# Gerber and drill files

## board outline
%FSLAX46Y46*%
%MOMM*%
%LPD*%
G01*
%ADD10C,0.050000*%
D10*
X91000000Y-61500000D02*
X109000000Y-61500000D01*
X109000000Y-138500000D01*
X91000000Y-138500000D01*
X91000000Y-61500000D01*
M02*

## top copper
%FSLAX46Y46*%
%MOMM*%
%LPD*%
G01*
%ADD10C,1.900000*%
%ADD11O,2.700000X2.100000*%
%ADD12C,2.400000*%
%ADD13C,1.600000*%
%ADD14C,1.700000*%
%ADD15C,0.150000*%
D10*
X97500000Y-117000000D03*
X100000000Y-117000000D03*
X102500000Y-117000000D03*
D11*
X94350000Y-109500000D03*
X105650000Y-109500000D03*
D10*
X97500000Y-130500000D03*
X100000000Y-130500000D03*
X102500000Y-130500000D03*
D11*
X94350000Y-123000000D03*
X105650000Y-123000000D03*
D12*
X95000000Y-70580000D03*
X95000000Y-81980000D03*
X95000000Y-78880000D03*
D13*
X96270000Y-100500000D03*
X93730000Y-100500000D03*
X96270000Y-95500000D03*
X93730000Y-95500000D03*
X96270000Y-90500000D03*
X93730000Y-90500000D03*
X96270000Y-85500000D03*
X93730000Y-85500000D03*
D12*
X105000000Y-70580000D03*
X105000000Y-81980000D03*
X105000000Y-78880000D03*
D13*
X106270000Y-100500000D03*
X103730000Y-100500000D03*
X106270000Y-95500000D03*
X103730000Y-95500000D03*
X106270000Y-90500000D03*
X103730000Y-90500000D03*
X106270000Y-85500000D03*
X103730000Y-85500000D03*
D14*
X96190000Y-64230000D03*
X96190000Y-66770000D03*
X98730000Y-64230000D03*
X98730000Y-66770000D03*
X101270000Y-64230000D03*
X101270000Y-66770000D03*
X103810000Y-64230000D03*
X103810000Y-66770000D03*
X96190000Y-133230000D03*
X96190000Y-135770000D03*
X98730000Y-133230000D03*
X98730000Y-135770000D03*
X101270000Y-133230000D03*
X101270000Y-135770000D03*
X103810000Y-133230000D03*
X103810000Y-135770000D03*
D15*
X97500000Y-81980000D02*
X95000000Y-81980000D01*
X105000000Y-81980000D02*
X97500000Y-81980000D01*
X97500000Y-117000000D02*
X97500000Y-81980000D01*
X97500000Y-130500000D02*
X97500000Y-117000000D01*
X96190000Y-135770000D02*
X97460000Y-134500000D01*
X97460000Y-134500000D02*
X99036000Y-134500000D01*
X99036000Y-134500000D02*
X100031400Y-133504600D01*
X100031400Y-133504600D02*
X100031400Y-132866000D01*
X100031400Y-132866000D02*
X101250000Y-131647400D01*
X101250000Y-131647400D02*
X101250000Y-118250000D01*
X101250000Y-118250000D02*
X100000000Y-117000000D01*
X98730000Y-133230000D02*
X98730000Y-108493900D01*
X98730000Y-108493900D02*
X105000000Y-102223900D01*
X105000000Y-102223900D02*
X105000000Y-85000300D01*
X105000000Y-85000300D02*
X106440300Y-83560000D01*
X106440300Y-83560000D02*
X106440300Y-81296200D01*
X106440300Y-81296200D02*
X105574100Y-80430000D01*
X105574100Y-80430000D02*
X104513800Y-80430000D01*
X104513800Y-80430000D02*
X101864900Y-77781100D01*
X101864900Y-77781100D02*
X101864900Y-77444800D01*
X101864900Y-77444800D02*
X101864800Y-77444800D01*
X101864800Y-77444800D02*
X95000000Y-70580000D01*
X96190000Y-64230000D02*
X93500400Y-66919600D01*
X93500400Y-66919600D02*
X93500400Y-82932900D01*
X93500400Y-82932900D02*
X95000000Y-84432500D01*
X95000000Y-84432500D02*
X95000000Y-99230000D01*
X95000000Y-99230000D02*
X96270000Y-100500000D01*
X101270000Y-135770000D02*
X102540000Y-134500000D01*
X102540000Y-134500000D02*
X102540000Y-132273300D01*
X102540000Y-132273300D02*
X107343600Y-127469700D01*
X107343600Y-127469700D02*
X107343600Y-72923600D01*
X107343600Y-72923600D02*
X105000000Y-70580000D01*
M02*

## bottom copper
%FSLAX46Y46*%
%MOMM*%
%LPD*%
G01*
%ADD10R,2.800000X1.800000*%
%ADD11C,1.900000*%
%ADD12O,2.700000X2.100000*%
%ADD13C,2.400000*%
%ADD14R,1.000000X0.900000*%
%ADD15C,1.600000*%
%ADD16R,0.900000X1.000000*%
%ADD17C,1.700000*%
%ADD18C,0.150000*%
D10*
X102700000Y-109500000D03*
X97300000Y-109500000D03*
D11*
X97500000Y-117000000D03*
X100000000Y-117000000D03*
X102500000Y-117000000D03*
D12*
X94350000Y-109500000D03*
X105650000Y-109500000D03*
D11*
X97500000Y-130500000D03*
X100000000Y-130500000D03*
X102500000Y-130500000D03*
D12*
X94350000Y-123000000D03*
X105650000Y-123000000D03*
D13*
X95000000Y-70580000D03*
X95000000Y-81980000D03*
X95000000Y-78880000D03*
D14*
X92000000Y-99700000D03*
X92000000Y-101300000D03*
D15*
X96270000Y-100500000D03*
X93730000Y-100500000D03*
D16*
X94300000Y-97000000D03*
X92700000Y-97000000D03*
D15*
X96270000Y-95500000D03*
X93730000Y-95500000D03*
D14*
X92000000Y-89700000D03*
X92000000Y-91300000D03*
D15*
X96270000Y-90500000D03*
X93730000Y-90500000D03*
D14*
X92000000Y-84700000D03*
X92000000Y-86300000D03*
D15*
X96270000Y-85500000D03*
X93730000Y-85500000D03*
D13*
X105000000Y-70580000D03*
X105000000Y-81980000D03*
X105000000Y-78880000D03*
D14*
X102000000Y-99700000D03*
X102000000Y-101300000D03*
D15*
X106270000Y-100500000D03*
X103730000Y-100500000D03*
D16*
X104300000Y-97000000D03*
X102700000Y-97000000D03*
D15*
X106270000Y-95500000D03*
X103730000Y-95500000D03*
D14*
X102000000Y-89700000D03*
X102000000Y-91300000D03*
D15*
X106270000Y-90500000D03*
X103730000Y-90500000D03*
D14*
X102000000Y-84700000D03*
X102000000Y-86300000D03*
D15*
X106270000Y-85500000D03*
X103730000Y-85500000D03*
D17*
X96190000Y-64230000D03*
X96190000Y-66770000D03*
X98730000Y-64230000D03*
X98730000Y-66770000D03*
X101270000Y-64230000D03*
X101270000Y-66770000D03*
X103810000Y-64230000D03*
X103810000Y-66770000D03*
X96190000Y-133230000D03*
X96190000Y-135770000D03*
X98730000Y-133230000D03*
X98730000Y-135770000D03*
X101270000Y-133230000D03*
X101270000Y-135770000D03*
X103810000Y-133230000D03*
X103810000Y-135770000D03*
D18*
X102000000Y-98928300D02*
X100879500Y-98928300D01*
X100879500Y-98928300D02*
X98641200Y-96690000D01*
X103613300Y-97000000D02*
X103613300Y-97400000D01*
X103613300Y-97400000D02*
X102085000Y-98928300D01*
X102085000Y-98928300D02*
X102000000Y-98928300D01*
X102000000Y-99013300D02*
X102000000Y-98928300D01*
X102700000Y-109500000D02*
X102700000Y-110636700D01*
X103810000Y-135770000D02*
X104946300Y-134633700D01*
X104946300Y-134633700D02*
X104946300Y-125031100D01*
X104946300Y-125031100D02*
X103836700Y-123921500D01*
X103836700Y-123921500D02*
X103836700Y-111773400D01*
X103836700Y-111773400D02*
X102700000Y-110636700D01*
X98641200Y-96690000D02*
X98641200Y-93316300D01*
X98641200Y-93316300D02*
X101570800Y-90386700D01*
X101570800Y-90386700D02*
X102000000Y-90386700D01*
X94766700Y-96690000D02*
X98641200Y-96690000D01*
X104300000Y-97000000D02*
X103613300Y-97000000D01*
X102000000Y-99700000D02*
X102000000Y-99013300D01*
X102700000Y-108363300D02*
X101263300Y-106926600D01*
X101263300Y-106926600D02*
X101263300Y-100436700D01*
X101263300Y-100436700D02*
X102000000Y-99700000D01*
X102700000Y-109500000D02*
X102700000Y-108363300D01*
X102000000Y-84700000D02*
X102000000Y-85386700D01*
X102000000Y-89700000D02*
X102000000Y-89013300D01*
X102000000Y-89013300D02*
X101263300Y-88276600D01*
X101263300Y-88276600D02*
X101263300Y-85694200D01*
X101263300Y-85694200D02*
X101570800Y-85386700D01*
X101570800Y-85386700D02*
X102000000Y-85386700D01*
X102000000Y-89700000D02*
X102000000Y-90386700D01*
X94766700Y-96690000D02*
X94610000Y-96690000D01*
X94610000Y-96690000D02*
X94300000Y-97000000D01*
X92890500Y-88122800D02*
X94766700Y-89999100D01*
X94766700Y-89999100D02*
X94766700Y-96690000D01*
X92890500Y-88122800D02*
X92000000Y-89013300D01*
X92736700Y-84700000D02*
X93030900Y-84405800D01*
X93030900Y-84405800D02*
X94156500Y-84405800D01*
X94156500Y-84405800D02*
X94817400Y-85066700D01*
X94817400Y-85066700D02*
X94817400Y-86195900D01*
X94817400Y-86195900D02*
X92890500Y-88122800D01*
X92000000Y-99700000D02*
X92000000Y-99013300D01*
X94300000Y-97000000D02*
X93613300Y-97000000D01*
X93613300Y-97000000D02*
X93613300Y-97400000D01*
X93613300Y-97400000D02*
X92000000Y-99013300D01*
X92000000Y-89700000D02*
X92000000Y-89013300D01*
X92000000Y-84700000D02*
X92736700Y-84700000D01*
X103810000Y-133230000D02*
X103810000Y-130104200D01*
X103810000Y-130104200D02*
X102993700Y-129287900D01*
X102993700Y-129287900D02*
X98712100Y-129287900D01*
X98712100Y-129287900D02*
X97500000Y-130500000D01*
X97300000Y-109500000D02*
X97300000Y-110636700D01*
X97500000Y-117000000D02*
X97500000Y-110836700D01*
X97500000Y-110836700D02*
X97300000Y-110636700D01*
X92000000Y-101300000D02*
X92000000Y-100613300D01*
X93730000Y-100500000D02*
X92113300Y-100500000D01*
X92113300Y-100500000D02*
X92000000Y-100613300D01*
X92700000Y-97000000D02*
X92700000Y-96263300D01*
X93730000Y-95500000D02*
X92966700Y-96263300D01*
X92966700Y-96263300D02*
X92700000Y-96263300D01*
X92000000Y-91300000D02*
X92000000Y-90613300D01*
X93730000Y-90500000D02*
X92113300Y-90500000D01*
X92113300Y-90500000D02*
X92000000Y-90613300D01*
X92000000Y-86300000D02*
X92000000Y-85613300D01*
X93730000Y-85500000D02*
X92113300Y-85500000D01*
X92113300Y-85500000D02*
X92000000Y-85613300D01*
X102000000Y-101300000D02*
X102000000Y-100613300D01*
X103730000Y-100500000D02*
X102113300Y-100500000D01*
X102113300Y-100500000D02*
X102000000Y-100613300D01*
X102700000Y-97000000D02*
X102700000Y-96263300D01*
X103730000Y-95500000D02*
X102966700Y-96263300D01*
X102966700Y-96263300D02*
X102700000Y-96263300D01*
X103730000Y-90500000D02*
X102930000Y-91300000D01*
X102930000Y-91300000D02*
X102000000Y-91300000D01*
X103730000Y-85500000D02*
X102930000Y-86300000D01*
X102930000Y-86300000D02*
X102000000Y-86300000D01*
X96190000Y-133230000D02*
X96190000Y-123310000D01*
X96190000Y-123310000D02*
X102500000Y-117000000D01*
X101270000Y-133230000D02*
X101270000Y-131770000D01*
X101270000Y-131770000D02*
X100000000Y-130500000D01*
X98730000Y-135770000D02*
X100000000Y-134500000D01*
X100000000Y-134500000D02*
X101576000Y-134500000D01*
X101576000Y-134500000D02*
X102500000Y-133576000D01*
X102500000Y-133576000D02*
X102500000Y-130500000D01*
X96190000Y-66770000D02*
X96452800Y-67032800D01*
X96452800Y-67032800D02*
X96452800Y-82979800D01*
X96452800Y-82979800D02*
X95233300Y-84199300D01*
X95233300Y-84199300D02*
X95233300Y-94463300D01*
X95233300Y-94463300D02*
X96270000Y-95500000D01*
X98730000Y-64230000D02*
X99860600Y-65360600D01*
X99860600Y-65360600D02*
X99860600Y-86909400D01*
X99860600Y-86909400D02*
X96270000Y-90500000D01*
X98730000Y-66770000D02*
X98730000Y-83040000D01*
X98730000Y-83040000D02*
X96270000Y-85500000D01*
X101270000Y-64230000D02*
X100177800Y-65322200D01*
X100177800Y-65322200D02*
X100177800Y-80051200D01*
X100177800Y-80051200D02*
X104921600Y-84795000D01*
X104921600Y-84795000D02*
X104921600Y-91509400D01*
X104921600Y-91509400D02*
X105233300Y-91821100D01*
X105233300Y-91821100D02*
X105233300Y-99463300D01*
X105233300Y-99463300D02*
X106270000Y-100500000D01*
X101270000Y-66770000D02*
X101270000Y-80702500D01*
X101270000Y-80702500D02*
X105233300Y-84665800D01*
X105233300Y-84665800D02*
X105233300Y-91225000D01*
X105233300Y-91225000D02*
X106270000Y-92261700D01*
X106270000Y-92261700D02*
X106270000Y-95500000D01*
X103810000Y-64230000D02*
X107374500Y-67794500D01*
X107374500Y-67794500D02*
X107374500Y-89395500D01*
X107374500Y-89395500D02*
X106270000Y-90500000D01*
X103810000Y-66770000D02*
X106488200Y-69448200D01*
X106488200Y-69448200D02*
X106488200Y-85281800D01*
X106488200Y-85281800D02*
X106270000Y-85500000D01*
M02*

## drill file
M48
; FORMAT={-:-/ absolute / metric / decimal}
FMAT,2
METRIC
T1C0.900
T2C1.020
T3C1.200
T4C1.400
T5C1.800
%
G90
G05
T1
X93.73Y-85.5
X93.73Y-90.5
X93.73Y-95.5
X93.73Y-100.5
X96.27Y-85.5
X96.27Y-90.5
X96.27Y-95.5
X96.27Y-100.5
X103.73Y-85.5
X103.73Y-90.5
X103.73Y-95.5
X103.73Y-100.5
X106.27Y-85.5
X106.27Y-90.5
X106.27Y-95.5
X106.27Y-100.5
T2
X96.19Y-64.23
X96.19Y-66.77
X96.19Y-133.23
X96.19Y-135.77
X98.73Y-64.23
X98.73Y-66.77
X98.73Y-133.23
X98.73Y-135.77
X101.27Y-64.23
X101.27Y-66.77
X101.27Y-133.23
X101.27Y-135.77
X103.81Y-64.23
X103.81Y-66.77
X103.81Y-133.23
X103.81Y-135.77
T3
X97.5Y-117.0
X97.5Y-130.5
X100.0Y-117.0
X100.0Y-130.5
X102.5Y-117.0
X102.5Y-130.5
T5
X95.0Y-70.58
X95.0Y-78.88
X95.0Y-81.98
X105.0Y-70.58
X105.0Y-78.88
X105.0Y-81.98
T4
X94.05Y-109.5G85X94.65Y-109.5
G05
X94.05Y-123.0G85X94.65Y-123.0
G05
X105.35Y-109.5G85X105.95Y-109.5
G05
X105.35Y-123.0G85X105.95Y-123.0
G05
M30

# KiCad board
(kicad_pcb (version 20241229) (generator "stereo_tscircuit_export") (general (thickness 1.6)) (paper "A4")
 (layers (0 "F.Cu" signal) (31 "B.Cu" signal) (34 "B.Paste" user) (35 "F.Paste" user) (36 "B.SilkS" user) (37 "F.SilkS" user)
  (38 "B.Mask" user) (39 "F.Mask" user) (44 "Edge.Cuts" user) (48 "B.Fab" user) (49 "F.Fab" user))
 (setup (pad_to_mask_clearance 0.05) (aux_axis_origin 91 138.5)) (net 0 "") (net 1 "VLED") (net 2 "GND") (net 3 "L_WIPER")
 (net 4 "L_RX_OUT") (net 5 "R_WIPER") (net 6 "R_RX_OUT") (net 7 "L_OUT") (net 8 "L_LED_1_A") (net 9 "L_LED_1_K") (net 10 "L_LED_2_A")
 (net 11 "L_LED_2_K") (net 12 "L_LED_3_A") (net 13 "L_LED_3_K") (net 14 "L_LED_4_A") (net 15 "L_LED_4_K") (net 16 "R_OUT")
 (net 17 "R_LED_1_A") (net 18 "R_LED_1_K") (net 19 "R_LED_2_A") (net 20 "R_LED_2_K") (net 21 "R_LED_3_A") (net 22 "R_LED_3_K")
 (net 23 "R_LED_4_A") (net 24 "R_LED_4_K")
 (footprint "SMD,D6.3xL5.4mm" (layer "B.Cu") (at 100 109.5)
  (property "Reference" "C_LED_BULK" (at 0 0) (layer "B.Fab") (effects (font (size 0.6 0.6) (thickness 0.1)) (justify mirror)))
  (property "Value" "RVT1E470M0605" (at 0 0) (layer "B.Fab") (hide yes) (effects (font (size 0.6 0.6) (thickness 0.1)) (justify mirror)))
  (pad "1" smd rect (at 2.700000 -0.000000 0) (size 2.8 1.8) (layers "B.Cu" "B.Paste" "B.Mask") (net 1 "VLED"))
  (pad "2" smd rect (at -2.700000 -0.000000 0) (size 2.8 1.8) (layers "B.Cu" "B.Paste" "B.Mask") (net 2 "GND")))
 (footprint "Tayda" (layer "F.Cu") (at 100 109.5)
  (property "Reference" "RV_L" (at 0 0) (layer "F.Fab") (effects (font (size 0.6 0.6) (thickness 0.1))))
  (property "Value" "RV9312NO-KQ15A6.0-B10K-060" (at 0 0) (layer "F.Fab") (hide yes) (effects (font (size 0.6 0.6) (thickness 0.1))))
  (pad "1" thru_hole circle (at -2.500000 7.500000 0) (size 1.9 1.9) (drill 1.2) (layers "*.Cu" "*.Mask") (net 2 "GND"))
  (pad "2" thru_hole circle (at 0.000000 7.500000 0) (size 1.9 1.9) (drill 1.2) (layers "*.Cu" "*.Mask") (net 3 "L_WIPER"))
  (pad "3" thru_hole circle (at 2.500000 7.500000 0) (size 1.9 1.9) (drill 1.2) (layers "*.Cu" "*.Mask") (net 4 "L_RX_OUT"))
  (pad "4" thru_hole oval (at -5.650000 -0.000000 0) (size 2.7 2.1) (drill oval 2 1.4) (layers "*.Cu" "*.Mask"))
  (pad "5" thru_hole oval (at 5.650000 -0.000000 0) (size 2.7 2.1) (drill oval 2 1.4) (layers "*.Cu" "*.Mask")))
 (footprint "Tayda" (layer "F.Cu") (at 100 123.0)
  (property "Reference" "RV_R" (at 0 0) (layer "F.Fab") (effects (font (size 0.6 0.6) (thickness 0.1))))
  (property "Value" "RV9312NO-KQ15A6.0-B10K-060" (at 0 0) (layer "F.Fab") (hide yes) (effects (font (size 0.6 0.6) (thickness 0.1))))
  (pad "1" thru_hole circle (at -2.500000 7.500000 0) (size 1.9 1.9) (drill 1.2) (layers "*.Cu" "*.Mask") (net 2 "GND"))
  (pad "2" thru_hole circle (at 0.000000 7.500000 0) (size 1.9 1.9) (drill 1.2) (layers "*.Cu" "*.Mask") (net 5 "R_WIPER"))
  (pad "3" thru_hole circle (at 2.500000 7.500000 0) (size 1.9 1.9) (drill 1.2) (layers "*.Cu" "*.Mask") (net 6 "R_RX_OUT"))
  (pad "4" thru_hole oval (at -5.650000 -0.000000 0) (size 2.7 2.1) (drill oval 2 1.4) (layers "*.Cu" "*.Mask"))
  (pad "5" thru_hole oval (at 5.650000 -0.000000 0) (size 2.7 2.1) (drill oval 2 1.4) (layers "*.Cu" "*.Mask")))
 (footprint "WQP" (layer "F.Cu") (at 95 75.5)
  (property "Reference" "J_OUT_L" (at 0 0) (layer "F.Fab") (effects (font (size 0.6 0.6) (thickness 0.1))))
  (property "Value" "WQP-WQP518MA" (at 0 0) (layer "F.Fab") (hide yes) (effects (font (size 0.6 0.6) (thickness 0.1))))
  (pad "1" thru_hole circle (at 0.000000 -4.920000 0) (size 2.4 2.4) (drill 1.8) (layers "*.Cu" "*.Mask") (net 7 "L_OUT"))
  (pad "2" thru_hole circle (at 0.000000 6.480000 0) (size 2.4 2.4) (drill 1.8) (layers "*.Cu" "*.Mask") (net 2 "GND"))
  (pad "3" thru_hole circle (at 0.000000 3.380000 0) (size 2.4 2.4) (drill 1.8) (layers "*.Cu" "*.Mask")))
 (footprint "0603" (layer "B.Cu") (at 92.0 100.5)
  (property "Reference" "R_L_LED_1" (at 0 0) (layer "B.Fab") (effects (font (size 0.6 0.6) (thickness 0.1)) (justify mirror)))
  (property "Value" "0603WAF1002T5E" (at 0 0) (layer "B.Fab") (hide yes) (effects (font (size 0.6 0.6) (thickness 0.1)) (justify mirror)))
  (pad "1" smd rect (at 0.000000 -0.800000 0) (size 1 0.9) (layers "B.Cu" "B.Paste" "B.Mask") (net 1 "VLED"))
  (pad "2" smd rect (at 0.000000 0.800000 0) (size 1 0.9) (layers "B.Cu" "B.Paste" "B.Mask") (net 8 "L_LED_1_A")))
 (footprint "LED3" (layer "F.Cu") (at 95 100.5)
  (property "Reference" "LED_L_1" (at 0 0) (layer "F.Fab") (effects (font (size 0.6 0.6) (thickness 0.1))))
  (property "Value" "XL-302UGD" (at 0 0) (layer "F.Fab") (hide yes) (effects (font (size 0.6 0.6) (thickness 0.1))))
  (pad "1" thru_hole circle (at 1.270000 -0.000000 0) (size 1.6 1.6) (drill 0.9) (layers "*.Cu" "*.Mask") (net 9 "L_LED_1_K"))
  (pad "2" thru_hole circle (at -1.270000 -0.000000 0) (size 1.6 1.6) (drill 0.9) (layers "*.Cu" "*.Mask") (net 8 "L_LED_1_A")))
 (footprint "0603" (layer "B.Cu") (at 93.5 97.0)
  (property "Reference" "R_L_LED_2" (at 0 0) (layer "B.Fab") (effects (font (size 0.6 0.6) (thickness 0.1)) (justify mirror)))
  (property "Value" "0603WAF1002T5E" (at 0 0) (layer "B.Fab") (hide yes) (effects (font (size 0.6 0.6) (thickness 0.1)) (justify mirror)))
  (pad "1" smd rect (at 0.800000 -0.000000 0) (size 0.9 1) (layers "B.Cu" "B.Paste" "B.Mask") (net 1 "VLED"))
  (pad "2" smd rect (at -0.800000 -0.000000 0) (size 0.9 1) (layers "B.Cu" "B.Paste" "B.Mask") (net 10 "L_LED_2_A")))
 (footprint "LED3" (layer "F.Cu") (at 95 95.5)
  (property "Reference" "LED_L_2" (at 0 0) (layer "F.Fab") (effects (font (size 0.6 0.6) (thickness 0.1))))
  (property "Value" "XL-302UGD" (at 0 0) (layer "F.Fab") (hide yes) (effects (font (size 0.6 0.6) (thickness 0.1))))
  (pad "1" thru_hole circle (at 1.270000 -0.000000 0) (size 1.6 1.6) (drill 0.9) (layers "*.Cu" "*.Mask") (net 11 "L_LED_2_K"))
  (pad "2" thru_hole circle (at -1.270000 -0.000000 0) (size 1.6 1.6) (drill 0.9) (layers "*.Cu" "*.Mask") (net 10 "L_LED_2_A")))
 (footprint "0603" (layer "B.Cu") (at 92.0 90.5)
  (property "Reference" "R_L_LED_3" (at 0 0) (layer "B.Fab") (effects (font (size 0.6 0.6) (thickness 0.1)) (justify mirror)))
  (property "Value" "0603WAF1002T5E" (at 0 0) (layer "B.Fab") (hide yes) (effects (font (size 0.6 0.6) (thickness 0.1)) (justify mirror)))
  (pad "1" smd rect (at 0.000000 -0.800000 0) (size 1 0.9) (layers "B.Cu" "B.Paste" "B.Mask") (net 1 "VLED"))
  (pad "2" smd rect (at 0.000000 0.800000 0) (size 1 0.9) (layers "B.Cu" "B.Paste" "B.Mask") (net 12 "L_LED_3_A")))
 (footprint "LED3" (layer "F.Cu") (at 95 90.5)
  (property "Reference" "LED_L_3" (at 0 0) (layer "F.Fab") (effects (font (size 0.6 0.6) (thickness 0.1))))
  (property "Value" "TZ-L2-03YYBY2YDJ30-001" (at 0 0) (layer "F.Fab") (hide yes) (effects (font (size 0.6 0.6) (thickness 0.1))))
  (pad "1" thru_hole circle (at 1.270000 -0.000000 0) (size 1.6 1.6) (drill 0.9) (layers "*.Cu" "*.Mask") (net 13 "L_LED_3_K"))
  (pad "2" thru_hole circle (at -1.270000 -0.000000 0) (size 1.6 1.6) (drill 0.9) (layers "*.Cu" "*.Mask") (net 12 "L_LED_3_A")))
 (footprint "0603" (layer "B.Cu") (at 92.0 85.5)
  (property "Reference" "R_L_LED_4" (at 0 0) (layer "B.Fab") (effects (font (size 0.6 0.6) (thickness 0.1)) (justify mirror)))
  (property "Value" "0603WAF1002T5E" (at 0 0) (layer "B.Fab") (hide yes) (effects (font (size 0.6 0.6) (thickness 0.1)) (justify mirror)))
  (pad "1" smd rect (at 0.000000 -0.800000 0) (size 1 0.9) (layers "B.Cu" "B.Paste" "B.Mask") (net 1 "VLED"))
  (pad "2" smd rect (at 0.000000 0.800000 0) (size 1 0.9) (layers "B.Cu" "B.Paste" "B.Mask") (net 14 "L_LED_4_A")))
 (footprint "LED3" (layer "F.Cu") (at 95 85.5)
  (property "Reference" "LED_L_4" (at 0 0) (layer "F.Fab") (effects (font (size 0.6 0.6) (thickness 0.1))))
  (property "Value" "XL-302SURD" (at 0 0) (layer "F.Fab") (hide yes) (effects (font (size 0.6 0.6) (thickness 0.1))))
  (pad "1" thru_hole circle (at 1.270000 -0.000000 0) (size 1.6 1.6) (drill 0.9) (layers "*.Cu" "*.Mask") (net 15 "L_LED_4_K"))
  (pad "2" thru_hole circle (at -1.270000 -0.000000 0) (size 1.6 1.6) (drill 0.9) (layers "*.Cu" "*.Mask") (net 14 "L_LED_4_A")))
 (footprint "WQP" (layer "F.Cu") (at 105 75.5)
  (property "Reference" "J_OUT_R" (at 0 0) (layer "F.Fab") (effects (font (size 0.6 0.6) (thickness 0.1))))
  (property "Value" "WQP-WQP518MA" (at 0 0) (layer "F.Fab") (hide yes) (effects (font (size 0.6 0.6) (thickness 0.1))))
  (pad "1" thru_hole circle (at 0.000000 -4.920000 0) (size 2.4 2.4) (drill 1.8) (layers "*.Cu" "*.Mask") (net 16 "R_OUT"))
  (pad "2" thru_hole circle (at 0.000000 6.480000 0) (size 2.4 2.4) (drill 1.8) (layers "*.Cu" "*.Mask") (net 2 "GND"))
  (pad "3" thru_hole circle (at 0.000000 3.380000 0) (size 2.4 2.4) (drill 1.8) (layers "*.Cu" "*.Mask")))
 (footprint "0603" (layer "B.Cu") (at 102.0 100.5)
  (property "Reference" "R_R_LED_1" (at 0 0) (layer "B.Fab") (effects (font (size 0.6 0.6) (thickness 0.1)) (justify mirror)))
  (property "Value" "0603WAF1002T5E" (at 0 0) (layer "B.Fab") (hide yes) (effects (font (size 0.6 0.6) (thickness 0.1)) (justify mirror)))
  (pad "1" smd rect (at 0.000000 -0.800000 0) (size 1 0.9) (layers "B.Cu" "B.Paste" "B.Mask") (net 1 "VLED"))
  (pad "2" smd rect (at 0.000000 0.800000 0) (size 1 0.9) (layers "B.Cu" "B.Paste" "B.Mask") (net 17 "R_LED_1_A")))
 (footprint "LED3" (layer "F.Cu") (at 105 100.5)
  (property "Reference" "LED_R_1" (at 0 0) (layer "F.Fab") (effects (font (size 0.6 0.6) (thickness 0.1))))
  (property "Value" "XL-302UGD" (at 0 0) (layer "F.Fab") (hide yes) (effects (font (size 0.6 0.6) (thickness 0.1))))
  (pad "1" thru_hole circle (at 1.270000 -0.000000 0) (size 1.6 1.6) (drill 0.9) (layers "*.Cu" "*.Mask") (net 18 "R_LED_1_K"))
  (pad "2" thru_hole circle (at -1.270000 -0.000000 0) (size 1.6 1.6) (drill 0.9) (layers "*.Cu" "*.Mask") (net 17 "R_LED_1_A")))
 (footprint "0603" (layer "B.Cu") (at 103.5 97.0)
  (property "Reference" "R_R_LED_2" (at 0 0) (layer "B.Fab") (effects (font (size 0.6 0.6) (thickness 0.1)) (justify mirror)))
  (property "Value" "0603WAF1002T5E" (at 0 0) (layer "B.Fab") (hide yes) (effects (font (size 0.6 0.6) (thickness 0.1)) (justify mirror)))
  (pad "1" smd rect (at 0.800000 -0.000000 0) (size 0.9 1) (layers "B.Cu" "B.Paste" "B.Mask") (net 1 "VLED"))
  (pad "2" smd rect (at -0.800000 -0.000000 0) (size 0.9 1) (layers "B.Cu" "B.Paste" "B.Mask") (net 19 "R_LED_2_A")))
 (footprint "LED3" (layer "F.Cu") (at 105 95.5)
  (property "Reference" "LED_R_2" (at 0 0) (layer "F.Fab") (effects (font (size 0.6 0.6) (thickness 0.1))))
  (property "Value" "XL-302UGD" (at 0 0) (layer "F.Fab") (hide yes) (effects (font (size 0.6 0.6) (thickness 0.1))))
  (pad "1" thru_hole circle (at 1.270000 -0.000000 0) (size 1.6 1.6) (drill 0.9) (layers "*.Cu" "*.Mask") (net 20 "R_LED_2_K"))
  (pad "2" thru_hole circle (at -1.270000 -0.000000 0) (size 1.6 1.6) (drill 0.9) (layers "*.Cu" "*.Mask") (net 19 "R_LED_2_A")))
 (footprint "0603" (layer "B.Cu") (at 102.0 90.5)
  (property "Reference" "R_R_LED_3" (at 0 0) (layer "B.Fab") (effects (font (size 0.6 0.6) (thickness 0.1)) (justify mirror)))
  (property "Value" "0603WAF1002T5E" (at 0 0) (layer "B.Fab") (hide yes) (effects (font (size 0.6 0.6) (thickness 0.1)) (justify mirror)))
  (pad "1" smd rect (at 0.000000 -0.800000 0) (size 1 0.9) (layers "B.Cu" "B.Paste" "B.Mask") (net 1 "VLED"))
  (pad "2" smd rect (at 0.000000 0.800000 0) (size 1 0.9) (layers "B.Cu" "B.Paste" "B.Mask") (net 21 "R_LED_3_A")))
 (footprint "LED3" (layer "F.Cu") (at 105 90.5)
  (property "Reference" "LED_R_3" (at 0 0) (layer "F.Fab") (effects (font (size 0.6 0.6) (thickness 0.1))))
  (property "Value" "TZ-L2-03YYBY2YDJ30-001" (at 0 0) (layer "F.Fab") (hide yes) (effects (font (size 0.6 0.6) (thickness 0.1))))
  (pad "1" thru_hole circle (at 1.270000 -0.000000 0) (size 1.6 1.6) (drill 0.9) (layers "*.Cu" "*.Mask") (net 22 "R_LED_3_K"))
  (pad "2" thru_hole circle (at -1.270000 -0.000000 0) (size 1.6 1.6) (drill 0.9) (layers "*.Cu" "*.Mask") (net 21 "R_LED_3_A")))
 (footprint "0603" (layer "B.Cu") (at 102.0 85.5)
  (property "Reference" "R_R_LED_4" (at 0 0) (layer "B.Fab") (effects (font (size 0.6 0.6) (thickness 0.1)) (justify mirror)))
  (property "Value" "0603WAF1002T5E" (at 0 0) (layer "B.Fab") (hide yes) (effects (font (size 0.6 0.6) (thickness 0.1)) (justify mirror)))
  (pad "1" smd rect (at 0.000000 -0.800000 0) (size 1 0.9) (layers "B.Cu" "B.Paste" "B.Mask") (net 1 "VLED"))
  (pad "2" smd rect (at 0.000000 0.800000 0) (size 1 0.9) (layers "B.Cu" "B.Paste" "B.Mask") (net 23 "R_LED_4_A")))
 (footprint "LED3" (layer "F.Cu") (at 105 85.5)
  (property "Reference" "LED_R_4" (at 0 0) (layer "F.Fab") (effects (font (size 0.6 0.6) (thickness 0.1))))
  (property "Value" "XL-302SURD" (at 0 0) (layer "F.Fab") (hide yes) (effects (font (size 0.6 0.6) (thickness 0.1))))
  (pad "1" thru_hole circle (at 1.270000 -0.000000 0) (size 1.6 1.6) (drill 0.9) (layers "*.Cu" "*.Mask") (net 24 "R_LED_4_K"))
  (pad "2" thru_hole circle (at -1.270000 -0.000000 0) (size 1.6 1.6) (drill 0.9) (layers "*.Cu" "*.Mask") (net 23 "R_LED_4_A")))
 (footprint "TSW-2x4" (layer "B.Cu") (at 100 65.5)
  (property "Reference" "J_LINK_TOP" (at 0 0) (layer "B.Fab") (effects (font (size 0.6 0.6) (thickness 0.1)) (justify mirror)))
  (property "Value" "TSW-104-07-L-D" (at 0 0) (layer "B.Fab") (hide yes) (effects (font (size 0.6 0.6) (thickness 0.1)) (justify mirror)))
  (pad "1" thru_hole circle (at -3.810000 -1.270000 0) (size 1.7 1.7) (drill 1.02) (layers "*.Cu" "*.Mask") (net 9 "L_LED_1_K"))
  (pad "2" thru_hole circle (at -3.810000 1.270000 0) (size 1.7 1.7) (drill 1.02) (layers "*.Cu" "*.Mask") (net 11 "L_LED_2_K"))
  (pad "3" thru_hole circle (at -1.270000 -1.270000 0) (size 1.7 1.7) (drill 1.02) (layers "*.Cu" "*.Mask") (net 13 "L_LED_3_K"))
  (pad "4" thru_hole circle (at -1.270000 1.270000 0) (size 1.7 1.7) (drill 1.02) (layers "*.Cu" "*.Mask") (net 15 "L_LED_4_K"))
  (pad "5" thru_hole circle (at 1.270000 -1.270000 0) (size 1.7 1.7) (drill 1.02) (layers "*.Cu" "*.Mask") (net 18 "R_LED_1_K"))
  (pad "6" thru_hole circle (at 1.270000 1.270000 0) (size 1.7 1.7) (drill 1.02) (layers "*.Cu" "*.Mask") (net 20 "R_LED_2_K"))
  (pad "7" thru_hole circle (at 3.810000 -1.270000 0) (size 1.7 1.7) (drill 1.02) (layers "*.Cu" "*.Mask") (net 22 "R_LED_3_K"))
  (pad "8" thru_hole circle (at 3.810000 1.270000 0) (size 1.7 1.7) (drill 1.02) (layers "*.Cu" "*.Mask") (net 24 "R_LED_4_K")))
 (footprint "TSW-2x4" (layer "B.Cu") (at 100 134.5)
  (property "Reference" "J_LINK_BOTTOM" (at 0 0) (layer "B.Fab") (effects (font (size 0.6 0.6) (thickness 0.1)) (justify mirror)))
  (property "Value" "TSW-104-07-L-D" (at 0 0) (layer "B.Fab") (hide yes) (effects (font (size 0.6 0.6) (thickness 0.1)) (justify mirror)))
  (pad "1" thru_hole circle (at -3.810000 -1.270000 0) (size 1.7 1.7) (drill 1.02) (layers "*.Cu" "*.Mask") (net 4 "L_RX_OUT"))
  (pad "2" thru_hole circle (at -3.810000 1.270000 0) (size 1.7 1.7) (drill 1.02) (layers "*.Cu" "*.Mask") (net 3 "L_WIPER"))
  (pad "3" thru_hole circle (at -1.270000 -1.270000 0) (size 1.7 1.7) (drill 1.02) (layers "*.Cu" "*.Mask") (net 7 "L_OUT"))
  (pad "4" thru_hole circle (at -1.270000 1.270000 0) (size 1.7 1.7) (drill 1.02) (layers "*.Cu" "*.Mask") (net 6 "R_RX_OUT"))
  (pad "5" thru_hole circle (at 1.270000 -1.270000 0) (size 1.7 1.7) (drill 1.02) (layers "*.Cu" "*.Mask") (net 5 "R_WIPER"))
  (pad "6" thru_hole circle (at 1.270000 1.270000 0) (size 1.7 1.7) (drill 1.02) (layers "*.Cu" "*.Mask") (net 16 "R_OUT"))
  (pad "7" thru_hole circle (at 3.810000 -1.270000 0) (size 1.7 1.7) (drill 1.02) (layers "*.Cu" "*.Mask") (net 2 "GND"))
  (pad "8" thru_hole circle (at 3.810000 1.270000 0) (size 1.7 1.7) (drill 1.02) (layers "*.Cu" "*.Mask") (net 1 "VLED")))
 (segment (start 102.000000 98.928300) (end 100.879500 98.928300) (width 0.15) (layer "B.Cu") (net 1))
 (segment (start 100.879500 98.928300) (end 98.641200 96.690000) (width 0.15) (layer "B.Cu") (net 1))
 (segment (start 103.613300 97.000000) (end 103.613300 97.400000) (width 0.15) (layer "B.Cu") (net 1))
 (segment (start 103.613300 97.400000) (end 102.085000 98.928300) (width 0.15) (layer "B.Cu") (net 1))
 (segment (start 102.085000 98.928300) (end 102.000000 98.928300) (width 0.15) (layer "B.Cu") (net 1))
 (segment (start 102.000000 99.013300) (end 102.000000 98.928300) (width 0.15) (layer "B.Cu") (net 1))
 (segment (start 102.700000 109.500000) (end 102.700000 110.636700) (width 0.15) (layer "B.Cu") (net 1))
 (segment (start 103.810000 135.770000) (end 104.946300 134.633700) (width 0.15) (layer "B.Cu") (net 1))
 (segment (start 104.946300 134.633700) (end 104.946300 125.031100) (width 0.15) (layer "B.Cu") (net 1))
 (segment (start 104.946300 125.031100) (end 103.836700 123.921500) (width 0.15) (layer "B.Cu") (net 1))
 (segment (start 103.836700 123.921500) (end 103.836700 111.773400) (width 0.15) (layer "B.Cu") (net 1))
 (segment (start 103.836700 111.773400) (end 102.700000 110.636700) (width 0.15) (layer "B.Cu") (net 1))
 (segment (start 98.641200 96.690000) (end 98.641200 93.316300) (width 0.15) (layer "B.Cu") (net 1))
 (segment (start 98.641200 93.316300) (end 101.570800 90.386700) (width 0.15) (layer "B.Cu") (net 1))
 (segment (start 101.570800 90.386700) (end 102.000000 90.386700) (width 0.15) (layer "B.Cu") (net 1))
 (segment (start 94.766700 96.690000) (end 98.641200 96.690000) (width 0.15) (layer "B.Cu") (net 1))
 (segment (start 104.300000 97.000000) (end 103.613300 97.000000) (width 0.15) (layer "B.Cu") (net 1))
 (segment (start 102.000000 99.700000) (end 102.000000 99.013300) (width 0.15) (layer "B.Cu") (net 1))
 (segment (start 102.700000 108.363300) (end 101.263300 106.926600) (width 0.15) (layer "B.Cu") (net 1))
 (segment (start 101.263300 106.926600) (end 101.263300 100.436700) (width 0.15) (layer "B.Cu") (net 1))
 (segment (start 101.263300 100.436700) (end 102.000000 99.700000) (width 0.15) (layer "B.Cu") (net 1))
 (segment (start 102.700000 109.500000) (end 102.700000 108.363300) (width 0.15) (layer "B.Cu") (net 1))
 (segment (start 102.000000 84.700000) (end 102.000000 85.386700) (width 0.15) (layer "B.Cu") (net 1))
 (segment (start 102.000000 89.700000) (end 102.000000 89.013300) (width 0.15) (layer "B.Cu") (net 1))
 (segment (start 102.000000 89.013300) (end 101.263300 88.276600) (width 0.15) (layer "B.Cu") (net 1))
 (segment (start 101.263300 88.276600) (end 101.263300 85.694200) (width 0.15) (layer "B.Cu") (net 1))
 (segment (start 101.263300 85.694200) (end 101.570800 85.386700) (width 0.15) (layer "B.Cu") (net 1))
 (segment (start 101.570800 85.386700) (end 102.000000 85.386700) (width 0.15) (layer "B.Cu") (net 1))
 (segment (start 102.000000 89.700000) (end 102.000000 90.386700) (width 0.15) (layer "B.Cu") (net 1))
 (segment (start 94.766700 96.690000) (end 94.610000 96.690000) (width 0.15) (layer "B.Cu") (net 1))
 (segment (start 94.610000 96.690000) (end 94.300000 97.000000) (width 0.15) (layer "B.Cu") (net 1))
 (segment (start 92.890500 88.122800) (end 94.766700 89.999100) (width 0.15) (layer "B.Cu") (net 1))
 (segment (start 94.766700 89.999100) (end 94.766700 96.690000) (width 0.15) (layer "B.Cu") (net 1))
 (segment (start 92.890500 88.122800) (end 92.000000 89.013300) (width 0.15) (layer "B.Cu") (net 1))
 (segment (start 92.736700 84.700000) (end 93.030900 84.405800) (width 0.15) (layer "B.Cu") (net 1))
 (segment (start 93.030900 84.405800) (end 94.156500 84.405800) (width 0.15) (layer "B.Cu") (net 1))
 (segment (start 94.156500 84.405800) (end 94.817400 85.066700) (width 0.15) (layer "B.Cu") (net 1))
 (segment (start 94.817400 85.066700) (end 94.817400 86.195900) (width 0.15) (layer "B.Cu") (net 1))
 (segment (start 94.817400 86.195900) (end 92.890500 88.122800) (width 0.15) (layer "B.Cu") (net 1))
 (segment (start 92.000000 99.700000) (end 92.000000 99.013300) (width 0.15) (layer "B.Cu") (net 1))
 (segment (start 94.300000 97.000000) (end 93.613300 97.000000) (width 0.15) (layer "B.Cu") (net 1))
 (segment (start 93.613300 97.000000) (end 93.613300 97.400000) (width 0.15) (layer "B.Cu") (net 1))
 (segment (start 93.613300 97.400000) (end 92.000000 99.013300) (width 0.15) (layer "B.Cu") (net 1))
 (segment (start 92.000000 89.700000) (end 92.000000 89.013300) (width 0.15) (layer "B.Cu") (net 1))
 (segment (start 92.000000 84.700000) (end 92.736700 84.700000) (width 0.15) (layer "B.Cu") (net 1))
 (segment (start 97.500000 81.980000) (end 95.000000 81.980000) (width 0.15) (layer "F.Cu") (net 2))
 (segment (start 105.000000 81.980000) (end 97.500000 81.980000) (width 0.15) (layer "F.Cu") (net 2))
 (segment (start 97.500000 117.000000) (end 97.500000 81.980000) (width 0.15) (layer "F.Cu") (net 2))
 (segment (start 103.810000 133.230000) (end 103.810000 130.104200) (width 0.15) (layer "B.Cu") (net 2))
 (segment (start 103.810000 130.104200) (end 102.993700 129.287900) (width 0.15) (layer "B.Cu") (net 2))
 (segment (start 102.993700 129.287900) (end 98.712100 129.287900) (width 0.15) (layer "B.Cu") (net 2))
 (segment (start 98.712100 129.287900) (end 97.500000 130.500000) (width 0.15) (layer "B.Cu") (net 2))
 (segment (start 97.300000 109.500000) (end 97.300000 110.636700) (width 0.15) (layer "B.Cu") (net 2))
 (segment (start 97.500000 117.000000) (end 97.500000 110.836700) (width 0.15) (layer "B.Cu") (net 2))
 (segment (start 97.500000 110.836700) (end 97.300000 110.636700) (width 0.15) (layer "B.Cu") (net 2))
 (segment (start 97.500000 130.500000) (end 97.500000 117.000000) (width 0.15) (layer "F.Cu") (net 2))
 (segment (start 92.000000 101.300000) (end 92.000000 100.613300) (width 0.15) (layer "B.Cu") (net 8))
 (segment (start 93.730000 100.500000) (end 92.113300 100.500000) (width 0.15) (layer "B.Cu") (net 8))
 (segment (start 92.113300 100.500000) (end 92.000000 100.613300) (width 0.15) (layer "B.Cu") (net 8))
 (segment (start 92.700000 97.000000) (end 92.700000 96.263300) (width 0.15) (layer "B.Cu") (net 10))
 (segment (start 93.730000 95.500000) (end 92.966700 96.263300) (width 0.15) (layer "B.Cu") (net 10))
 (segment (start 92.966700 96.263300) (end 92.700000 96.263300) (width 0.15) (layer "B.Cu") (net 10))
 (segment (start 92.000000 91.300000) (end 92.000000 90.613300) (width 0.15) (layer "B.Cu") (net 12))
 (segment (start 93.730000 90.500000) (end 92.113300 90.500000) (width 0.15) (layer "B.Cu") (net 12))
 (segment (start 92.113300 90.500000) (end 92.000000 90.613300) (width 0.15) (layer "B.Cu") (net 12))
 (segment (start 92.000000 86.300000) (end 92.000000 85.613300) (width 0.15) (layer "B.Cu") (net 14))
 (segment (start 93.730000 85.500000) (end 92.113300 85.500000) (width 0.15) (layer "B.Cu") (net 14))
 (segment (start 92.113300 85.500000) (end 92.000000 85.613300) (width 0.15) (layer "B.Cu") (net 14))
 (segment (start 102.000000 101.300000) (end 102.000000 100.613300) (width 0.15) (layer "B.Cu") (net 17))
 (segment (start 103.730000 100.500000) (end 102.113300 100.500000) (width 0.15) (layer "B.Cu") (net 17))
 (segment (start 102.113300 100.500000) (end 102.000000 100.613300) (width 0.15) (layer "B.Cu") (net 17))
 (segment (start 102.700000 97.000000) (end 102.700000 96.263300) (width 0.15) (layer "B.Cu") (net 19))
 (segment (start 103.730000 95.500000) (end 102.966700 96.263300) (width 0.15) (layer "B.Cu") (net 19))
 (segment (start 102.966700 96.263300) (end 102.700000 96.263300) (width 0.15) (layer "B.Cu") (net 19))
 (segment (start 103.730000 90.500000) (end 102.930000 91.300000) (width 0.15) (layer "B.Cu") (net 21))
 (segment (start 102.930000 91.300000) (end 102.000000 91.300000) (width 0.15) (layer "B.Cu") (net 21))
 (segment (start 103.730000 85.500000) (end 102.930000 86.300000) (width 0.15) (layer "B.Cu") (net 23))
 (segment (start 102.930000 86.300000) (end 102.000000 86.300000) (width 0.15) (layer "B.Cu") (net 23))
 (segment (start 96.190000 135.770000) (end 97.460000 134.500000) (width 0.15) (layer "F.Cu") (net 3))
 (segment (start 97.460000 134.500000) (end 99.036000 134.500000) (width 0.15) (layer "F.Cu") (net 3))
 (segment (start 99.036000 134.500000) (end 100.031400 133.504600) (width 0.15) (layer "F.Cu") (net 3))
 (segment (start 100.031400 133.504600) (end 100.031400 132.866000) (width 0.15) (layer "F.Cu") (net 3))
 (segment (start 100.031400 132.866000) (end 101.250000 131.647400) (width 0.15) (layer "F.Cu") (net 3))
 (segment (start 101.250000 131.647400) (end 101.250000 118.250000) (width 0.15) (layer "F.Cu") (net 3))
 (segment (start 101.250000 118.250000) (end 100.000000 117.000000) (width 0.15) (layer "F.Cu") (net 3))
 (segment (start 96.190000 133.230000) (end 96.190000 123.310000) (width 0.15) (layer "B.Cu") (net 4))
 (segment (start 96.190000 123.310000) (end 102.500000 117.000000) (width 0.15) (layer "B.Cu") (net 4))
 (segment (start 101.270000 133.230000) (end 101.270000 131.770000) (width 0.15) (layer "B.Cu") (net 5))
 (segment (start 101.270000 131.770000) (end 100.000000 130.500000) (width 0.15) (layer "B.Cu") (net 5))
 (segment (start 98.730000 135.770000) (end 100.000000 134.500000) (width 0.15) (layer "B.Cu") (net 6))
 (segment (start 100.000000 134.500000) (end 101.576000 134.500000) (width 0.15) (layer "B.Cu") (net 6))
 (segment (start 101.576000 134.500000) (end 102.500000 133.576000) (width 0.15) (layer "B.Cu") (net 6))
 (segment (start 102.500000 133.576000) (end 102.500000 130.500000) (width 0.15) (layer "B.Cu") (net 6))
 (segment (start 98.730000 133.230000) (end 98.730000 108.493900) (width 0.15) (layer "F.Cu") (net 7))
 (segment (start 98.730000 108.493900) (end 105.000000 102.223900) (width 0.15) (layer "F.Cu") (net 7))
 (segment (start 105.000000 102.223900) (end 105.000000 85.000300) (width 0.15) (layer "F.Cu") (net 7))
 (segment (start 105.000000 85.000300) (end 106.440300 83.560000) (width 0.15) (layer "F.Cu") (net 7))
 (segment (start 106.440300 83.560000) (end 106.440300 81.296200) (width 0.15) (layer "F.Cu") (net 7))
 (segment (start 106.440300 81.296200) (end 105.574100 80.430000) (width 0.15) (layer "F.Cu") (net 7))
 (segment (start 105.574100 80.430000) (end 104.513800 80.430000) (width 0.15) (layer "F.Cu") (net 7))
 (segment (start 104.513800 80.430000) (end 101.864900 77.781100) (width 0.15) (layer "F.Cu") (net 7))
 (segment (start 101.864900 77.781100) (end 101.864900 77.444800) (width 0.15) (layer "F.Cu") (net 7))
 (segment (start 101.864900 77.444800) (end 101.864800 77.444800) (width 0.15) (layer "F.Cu") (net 7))
 (segment (start 101.864800 77.444800) (end 95.000000 70.580000) (width 0.15) (layer "F.Cu") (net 7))
 (segment (start 96.190000 64.230000) (end 93.500400 66.919600) (width 0.15) (layer "F.Cu") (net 9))
 (segment (start 93.500400 66.919600) (end 93.500400 82.932900) (width 0.15) (layer "F.Cu") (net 9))
 (segment (start 93.500400 82.932900) (end 95.000000 84.432500) (width 0.15) (layer "F.Cu") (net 9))
 (segment (start 95.000000 84.432500) (end 95.000000 99.230000) (width 0.15) (layer "F.Cu") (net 9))
 (segment (start 95.000000 99.230000) (end 96.270000 100.500000) (width 0.15) (layer "F.Cu") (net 9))
 (segment (start 96.190000 66.770000) (end 96.452800 67.032800) (width 0.15) (layer "B.Cu") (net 11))
 (segment (start 96.452800 67.032800) (end 96.452800 82.979800) (width 0.15) (layer "B.Cu") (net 11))
 (segment (start 96.452800 82.979800) (end 95.233300 84.199300) (width 0.15) (layer "B.Cu") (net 11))
 (segment (start 95.233300 84.199300) (end 95.233300 94.463300) (width 0.15) (layer "B.Cu") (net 11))
 (segment (start 95.233300 94.463300) (end 96.270000 95.500000) (width 0.15) (layer "B.Cu") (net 11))
 (segment (start 98.730000 64.230000) (end 99.860600 65.360600) (width 0.15) (layer "B.Cu") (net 13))
 (segment (start 99.860600 65.360600) (end 99.860600 86.909400) (width 0.15) (layer "B.Cu") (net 13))
 (segment (start 99.860600 86.909400) (end 96.270000 90.500000) (width 0.15) (layer "B.Cu") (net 13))
 (segment (start 98.730000 66.770000) (end 98.730000 83.040000) (width 0.15) (layer "B.Cu") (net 15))
 (segment (start 98.730000 83.040000) (end 96.270000 85.500000) (width 0.15) (layer "B.Cu") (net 15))
 (segment (start 101.270000 135.770000) (end 102.540000 134.500000) (width 0.15) (layer "F.Cu") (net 16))
 (segment (start 102.540000 134.500000) (end 102.540000 132.273300) (width 0.15) (layer "F.Cu") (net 16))
 (segment (start 102.540000 132.273300) (end 107.343600 127.469700) (width 0.15) (layer "F.Cu") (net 16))
 (segment (start 107.343600 127.469700) (end 107.343600 72.923600) (width 0.15) (layer "F.Cu") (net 16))
 (segment (start 107.343600 72.923600) (end 105.000000 70.580000) (width 0.15) (layer "F.Cu") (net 16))
 (segment (start 101.270000 64.230000) (end 100.177800 65.322200) (width 0.15) (layer "B.Cu") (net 18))
 (segment (start 100.177800 65.322200) (end 100.177800 80.051200) (width 0.15) (layer "B.Cu") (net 18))
 (segment (start 100.177800 80.051200) (end 104.921600 84.795000) (width 0.15) (layer "B.Cu") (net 18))
 (segment (start 104.921600 84.795000) (end 104.921600 91.509400) (width 0.15) (layer "B.Cu") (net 18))
 (segment (start 104.921600 91.509400) (end 105.233300 91.821100) (width 0.15) (layer "B.Cu") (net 18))
 (segment (start 105.233300 91.821100) (end 105.233300 99.463300) (width 0.15) (layer "B.Cu") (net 18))
 (segment (start 105.233300 99.463300) (end 106.270000 100.500000) (width 0.15) (layer "B.Cu") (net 18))
 (segment (start 101.270000 66.770000) (end 101.270000 80.702500) (width 0.15) (layer "B.Cu") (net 20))
 (segment (start 101.270000 80.702500) (end 105.233300 84.665800) (width 0.15) (layer "B.Cu") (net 20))
 (segment (start 105.233300 84.665800) (end 105.233300 91.225000) (width 0.15) (layer "B.Cu") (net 20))
 (segment (start 105.233300 91.225000) (end 106.270000 92.261700) (width 0.15) (layer "B.Cu") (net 20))
 (segment (start 106.270000 92.261700) (end 106.270000 95.500000) (width 0.15) (layer "B.Cu") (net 20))
 (segment (start 103.810000 64.230000) (end 107.374500 67.794500) (width 0.15) (layer "B.Cu") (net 22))
 (segment (start 107.374500 67.794500) (end 107.374500 89.395500) (width 0.15) (layer "B.Cu") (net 22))
 (segment (start 107.374500 89.395500) (end 106.270000 90.500000) (width 0.15) (layer "B.Cu") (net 22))
 (segment (start 103.810000 66.770000) (end 106.488200 69.448200) (width 0.15) (layer "B.Cu") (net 24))
 (segment (start 106.488200 69.448200) (end 106.488200 85.281800) (width 0.15) (layer "B.Cu") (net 24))
 (segment (start 106.488200 85.281800) (end 106.270000 85.500000) (width 0.15) (layer "B.Cu") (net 24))
 (gr_rect (start 91.0 61.5) (end 109.0 138.5) (stroke (width 0.05) (type default)) (fill none) (layer "Edge.Cuts")))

